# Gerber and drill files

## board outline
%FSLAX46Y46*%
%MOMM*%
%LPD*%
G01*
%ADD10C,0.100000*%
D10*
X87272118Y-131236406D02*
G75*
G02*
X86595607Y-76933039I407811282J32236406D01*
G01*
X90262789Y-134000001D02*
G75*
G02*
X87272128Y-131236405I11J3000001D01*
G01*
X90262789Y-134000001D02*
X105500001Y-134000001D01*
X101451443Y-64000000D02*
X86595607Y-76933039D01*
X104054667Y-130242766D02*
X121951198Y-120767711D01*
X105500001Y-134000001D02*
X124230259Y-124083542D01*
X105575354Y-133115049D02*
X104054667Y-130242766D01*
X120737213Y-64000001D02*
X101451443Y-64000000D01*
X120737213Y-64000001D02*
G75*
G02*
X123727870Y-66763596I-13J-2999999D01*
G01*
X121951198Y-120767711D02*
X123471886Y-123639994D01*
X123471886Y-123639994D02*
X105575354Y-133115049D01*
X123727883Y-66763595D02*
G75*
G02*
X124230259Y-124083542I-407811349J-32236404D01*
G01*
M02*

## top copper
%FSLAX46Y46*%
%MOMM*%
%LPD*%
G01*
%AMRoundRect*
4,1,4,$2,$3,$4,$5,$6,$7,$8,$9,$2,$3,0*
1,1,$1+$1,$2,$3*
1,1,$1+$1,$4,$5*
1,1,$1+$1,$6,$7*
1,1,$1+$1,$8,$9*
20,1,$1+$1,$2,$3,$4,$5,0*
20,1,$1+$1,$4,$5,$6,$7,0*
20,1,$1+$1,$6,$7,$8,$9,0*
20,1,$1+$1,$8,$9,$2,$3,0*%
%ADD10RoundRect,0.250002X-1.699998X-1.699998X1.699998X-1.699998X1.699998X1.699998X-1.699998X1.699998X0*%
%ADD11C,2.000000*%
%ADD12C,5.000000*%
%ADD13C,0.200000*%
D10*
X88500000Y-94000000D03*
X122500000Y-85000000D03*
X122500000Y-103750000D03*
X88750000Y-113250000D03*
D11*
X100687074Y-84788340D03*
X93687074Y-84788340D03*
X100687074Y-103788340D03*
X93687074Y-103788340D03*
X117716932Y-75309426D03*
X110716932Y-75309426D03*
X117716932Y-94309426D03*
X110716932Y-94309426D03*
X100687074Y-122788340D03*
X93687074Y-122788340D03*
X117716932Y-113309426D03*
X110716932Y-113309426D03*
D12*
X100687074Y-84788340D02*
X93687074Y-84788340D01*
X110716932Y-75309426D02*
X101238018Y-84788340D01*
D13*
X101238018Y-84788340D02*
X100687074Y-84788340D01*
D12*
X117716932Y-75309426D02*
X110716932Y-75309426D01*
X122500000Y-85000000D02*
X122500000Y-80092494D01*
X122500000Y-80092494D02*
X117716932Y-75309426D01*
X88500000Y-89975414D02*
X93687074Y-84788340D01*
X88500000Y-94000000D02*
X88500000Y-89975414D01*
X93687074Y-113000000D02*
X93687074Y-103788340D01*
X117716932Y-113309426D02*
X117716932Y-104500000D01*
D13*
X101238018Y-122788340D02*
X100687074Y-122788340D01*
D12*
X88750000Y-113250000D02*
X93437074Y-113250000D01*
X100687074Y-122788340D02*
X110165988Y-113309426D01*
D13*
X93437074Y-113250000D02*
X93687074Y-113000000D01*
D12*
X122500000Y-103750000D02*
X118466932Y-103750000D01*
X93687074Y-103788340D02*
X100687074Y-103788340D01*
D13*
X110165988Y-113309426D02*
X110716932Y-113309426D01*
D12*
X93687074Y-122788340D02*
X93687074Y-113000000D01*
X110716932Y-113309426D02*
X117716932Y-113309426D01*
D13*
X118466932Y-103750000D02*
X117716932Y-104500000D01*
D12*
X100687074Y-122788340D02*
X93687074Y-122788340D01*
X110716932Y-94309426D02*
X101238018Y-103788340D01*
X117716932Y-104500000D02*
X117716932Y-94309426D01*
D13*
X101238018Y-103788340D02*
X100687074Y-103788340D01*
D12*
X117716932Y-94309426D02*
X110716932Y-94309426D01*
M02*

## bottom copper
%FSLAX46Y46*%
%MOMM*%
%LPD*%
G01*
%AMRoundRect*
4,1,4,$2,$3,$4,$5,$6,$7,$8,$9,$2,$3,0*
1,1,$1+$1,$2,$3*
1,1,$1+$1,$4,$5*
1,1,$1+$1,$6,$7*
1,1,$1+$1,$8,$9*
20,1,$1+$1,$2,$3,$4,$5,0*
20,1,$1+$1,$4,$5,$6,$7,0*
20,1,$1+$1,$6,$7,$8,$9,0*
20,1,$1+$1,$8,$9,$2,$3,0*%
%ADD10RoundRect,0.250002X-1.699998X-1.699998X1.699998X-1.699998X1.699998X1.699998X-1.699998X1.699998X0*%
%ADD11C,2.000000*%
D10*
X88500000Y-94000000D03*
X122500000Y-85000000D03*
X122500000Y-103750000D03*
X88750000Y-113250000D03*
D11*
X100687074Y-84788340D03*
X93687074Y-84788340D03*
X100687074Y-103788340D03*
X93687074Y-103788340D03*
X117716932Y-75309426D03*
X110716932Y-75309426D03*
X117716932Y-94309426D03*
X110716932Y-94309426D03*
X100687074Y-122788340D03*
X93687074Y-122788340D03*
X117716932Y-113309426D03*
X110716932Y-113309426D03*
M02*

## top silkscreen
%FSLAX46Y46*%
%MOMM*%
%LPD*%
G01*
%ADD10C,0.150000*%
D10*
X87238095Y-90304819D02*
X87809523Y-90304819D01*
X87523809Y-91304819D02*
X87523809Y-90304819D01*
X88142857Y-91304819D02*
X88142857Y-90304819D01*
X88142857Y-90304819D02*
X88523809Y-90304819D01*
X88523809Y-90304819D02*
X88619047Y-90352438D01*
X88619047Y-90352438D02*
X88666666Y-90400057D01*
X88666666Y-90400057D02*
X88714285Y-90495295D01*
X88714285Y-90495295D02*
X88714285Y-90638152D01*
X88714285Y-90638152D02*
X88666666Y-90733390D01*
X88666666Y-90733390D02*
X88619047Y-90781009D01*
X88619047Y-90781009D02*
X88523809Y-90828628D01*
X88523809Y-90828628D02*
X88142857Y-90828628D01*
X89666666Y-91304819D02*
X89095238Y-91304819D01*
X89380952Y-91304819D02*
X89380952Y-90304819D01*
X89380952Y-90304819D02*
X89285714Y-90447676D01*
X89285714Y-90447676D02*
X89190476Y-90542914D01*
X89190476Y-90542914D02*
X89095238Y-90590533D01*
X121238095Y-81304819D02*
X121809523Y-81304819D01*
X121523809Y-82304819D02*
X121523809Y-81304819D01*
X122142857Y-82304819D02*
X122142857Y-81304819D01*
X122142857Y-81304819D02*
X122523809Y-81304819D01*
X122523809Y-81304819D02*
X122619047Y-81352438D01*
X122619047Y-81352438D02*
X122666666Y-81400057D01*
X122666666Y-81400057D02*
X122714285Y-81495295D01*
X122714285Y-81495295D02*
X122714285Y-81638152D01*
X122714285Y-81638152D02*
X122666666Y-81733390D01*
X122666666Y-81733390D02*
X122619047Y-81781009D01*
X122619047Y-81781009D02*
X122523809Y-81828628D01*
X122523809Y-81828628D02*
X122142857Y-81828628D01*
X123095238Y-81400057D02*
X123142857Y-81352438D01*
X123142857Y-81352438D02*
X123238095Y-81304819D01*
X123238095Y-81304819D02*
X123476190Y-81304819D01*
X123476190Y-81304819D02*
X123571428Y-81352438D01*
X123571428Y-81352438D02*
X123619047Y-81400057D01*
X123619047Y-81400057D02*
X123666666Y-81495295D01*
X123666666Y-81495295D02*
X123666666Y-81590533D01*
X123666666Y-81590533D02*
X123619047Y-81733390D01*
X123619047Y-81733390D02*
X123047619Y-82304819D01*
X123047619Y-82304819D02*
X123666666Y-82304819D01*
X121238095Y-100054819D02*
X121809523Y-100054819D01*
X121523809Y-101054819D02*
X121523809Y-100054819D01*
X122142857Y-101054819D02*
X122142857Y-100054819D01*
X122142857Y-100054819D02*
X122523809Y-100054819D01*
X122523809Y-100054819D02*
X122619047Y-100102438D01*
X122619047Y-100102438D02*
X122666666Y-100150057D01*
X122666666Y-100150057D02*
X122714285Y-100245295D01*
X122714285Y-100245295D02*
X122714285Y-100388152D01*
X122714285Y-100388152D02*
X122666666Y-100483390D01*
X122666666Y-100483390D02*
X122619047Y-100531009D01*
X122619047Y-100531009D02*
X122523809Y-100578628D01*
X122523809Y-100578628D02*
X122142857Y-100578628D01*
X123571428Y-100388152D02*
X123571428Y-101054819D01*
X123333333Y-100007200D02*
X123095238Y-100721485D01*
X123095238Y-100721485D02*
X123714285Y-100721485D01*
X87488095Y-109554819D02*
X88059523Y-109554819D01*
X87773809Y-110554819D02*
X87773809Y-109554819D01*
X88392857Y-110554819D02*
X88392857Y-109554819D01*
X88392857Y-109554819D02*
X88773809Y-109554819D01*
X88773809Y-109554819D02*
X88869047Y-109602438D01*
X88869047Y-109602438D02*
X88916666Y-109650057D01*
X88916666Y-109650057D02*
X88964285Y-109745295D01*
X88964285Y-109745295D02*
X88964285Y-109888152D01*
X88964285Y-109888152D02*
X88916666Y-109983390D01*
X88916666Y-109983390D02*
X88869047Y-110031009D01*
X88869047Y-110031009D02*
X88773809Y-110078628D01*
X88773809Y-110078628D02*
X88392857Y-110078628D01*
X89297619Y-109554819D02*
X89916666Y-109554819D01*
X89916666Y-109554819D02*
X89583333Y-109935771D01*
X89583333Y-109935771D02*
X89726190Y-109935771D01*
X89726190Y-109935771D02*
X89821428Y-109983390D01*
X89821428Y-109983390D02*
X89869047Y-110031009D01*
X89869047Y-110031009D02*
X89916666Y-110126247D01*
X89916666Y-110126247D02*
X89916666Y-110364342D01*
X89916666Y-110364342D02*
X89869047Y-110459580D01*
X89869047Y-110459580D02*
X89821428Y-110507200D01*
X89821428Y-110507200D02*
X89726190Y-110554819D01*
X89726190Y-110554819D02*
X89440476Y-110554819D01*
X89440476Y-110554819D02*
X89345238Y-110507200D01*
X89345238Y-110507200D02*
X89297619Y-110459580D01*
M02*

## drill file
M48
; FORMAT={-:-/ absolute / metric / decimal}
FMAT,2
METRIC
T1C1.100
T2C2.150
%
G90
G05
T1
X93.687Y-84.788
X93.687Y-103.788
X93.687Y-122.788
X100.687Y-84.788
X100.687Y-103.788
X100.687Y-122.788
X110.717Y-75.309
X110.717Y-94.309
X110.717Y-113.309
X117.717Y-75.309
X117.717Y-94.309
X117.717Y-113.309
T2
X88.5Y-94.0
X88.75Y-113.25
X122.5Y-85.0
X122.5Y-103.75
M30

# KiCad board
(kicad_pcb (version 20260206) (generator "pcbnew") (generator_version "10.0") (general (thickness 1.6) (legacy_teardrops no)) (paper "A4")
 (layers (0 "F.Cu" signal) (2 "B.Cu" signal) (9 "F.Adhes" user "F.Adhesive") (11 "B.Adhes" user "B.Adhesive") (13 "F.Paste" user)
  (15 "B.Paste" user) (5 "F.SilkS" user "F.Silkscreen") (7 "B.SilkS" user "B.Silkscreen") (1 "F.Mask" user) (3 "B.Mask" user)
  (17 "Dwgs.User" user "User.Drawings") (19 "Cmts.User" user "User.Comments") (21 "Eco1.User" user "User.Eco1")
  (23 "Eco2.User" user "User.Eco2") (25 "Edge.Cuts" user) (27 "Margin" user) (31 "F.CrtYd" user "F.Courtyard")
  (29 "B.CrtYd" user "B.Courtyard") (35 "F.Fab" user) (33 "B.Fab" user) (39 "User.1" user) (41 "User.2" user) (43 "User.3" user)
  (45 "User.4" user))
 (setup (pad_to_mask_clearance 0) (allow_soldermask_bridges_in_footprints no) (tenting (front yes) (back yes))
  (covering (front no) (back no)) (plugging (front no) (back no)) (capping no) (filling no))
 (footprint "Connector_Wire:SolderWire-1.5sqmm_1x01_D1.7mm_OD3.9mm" (layer "F.Cu") (at 88.5 94)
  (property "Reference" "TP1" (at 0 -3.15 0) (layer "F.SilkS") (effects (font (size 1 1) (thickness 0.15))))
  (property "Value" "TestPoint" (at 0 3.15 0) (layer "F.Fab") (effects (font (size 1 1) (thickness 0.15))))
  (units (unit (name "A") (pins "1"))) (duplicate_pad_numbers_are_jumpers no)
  (pad "1" thru_hole roundrect (at 0 0) (size 3.9 3.9) (drill 2.15) (layers "*.Cu" "*.Mask") (remove_unused_layers no)
   (roundrect_rratio 0.064103) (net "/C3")))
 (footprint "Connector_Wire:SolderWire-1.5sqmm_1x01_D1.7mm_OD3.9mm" (layer "F.Cu") (at 122.5 85)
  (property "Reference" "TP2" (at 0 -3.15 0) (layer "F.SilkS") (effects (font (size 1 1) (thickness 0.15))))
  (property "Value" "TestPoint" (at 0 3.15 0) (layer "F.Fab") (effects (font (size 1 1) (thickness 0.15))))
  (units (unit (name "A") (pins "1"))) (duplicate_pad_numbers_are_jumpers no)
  (pad "1" thru_hole roundrect (at 0 0) (size 3.9 3.9) (drill 2.15) (layers "*.Cu" "*.Mask") (remove_unused_layers no)
   (roundrect_rratio 0.064103) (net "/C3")))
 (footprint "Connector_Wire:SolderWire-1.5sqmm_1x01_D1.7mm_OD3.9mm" (layer "F.Cu") (at 122.5 103.75)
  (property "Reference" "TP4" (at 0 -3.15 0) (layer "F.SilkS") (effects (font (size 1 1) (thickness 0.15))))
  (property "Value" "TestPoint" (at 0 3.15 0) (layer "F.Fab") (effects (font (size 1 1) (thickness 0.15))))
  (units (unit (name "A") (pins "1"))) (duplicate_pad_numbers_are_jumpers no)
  (pad "1" thru_hole roundrect (at 0 0) (size 3.9 3.9) (drill 2.15) (layers "*.Cu" "*.Mask") (remove_unused_layers no)
   (roundrect_rratio 0.064103) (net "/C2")))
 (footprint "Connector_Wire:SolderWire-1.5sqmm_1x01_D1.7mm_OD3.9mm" (layer "F.Cu") (at 88.75 113.25)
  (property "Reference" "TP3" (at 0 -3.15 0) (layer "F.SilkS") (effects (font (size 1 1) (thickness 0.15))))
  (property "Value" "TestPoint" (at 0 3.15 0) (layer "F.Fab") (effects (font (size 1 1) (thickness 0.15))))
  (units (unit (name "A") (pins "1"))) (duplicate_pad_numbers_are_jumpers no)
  (pad "1" thru_hole roundrect (at 0 0) (size 3.9 3.9) (drill 2.15) (layers "*.Cu" "*.Mask") (remove_unused_layers no)
   (roundrect_rratio 0.064103) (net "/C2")))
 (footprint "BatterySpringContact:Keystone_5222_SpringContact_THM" (layer "B.Cu") (at 97.187074 84.78834 180)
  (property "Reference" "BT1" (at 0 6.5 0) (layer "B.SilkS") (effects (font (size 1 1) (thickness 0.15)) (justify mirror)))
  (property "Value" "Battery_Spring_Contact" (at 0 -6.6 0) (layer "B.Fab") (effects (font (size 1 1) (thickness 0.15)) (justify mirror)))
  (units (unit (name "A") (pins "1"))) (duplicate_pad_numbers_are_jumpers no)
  (pad "1" thru_hole circle (at -3.5 0 180) (size 2 2) (drill 1.1) (layers "*.Cu" "*.Mask") (remove_unused_layers no) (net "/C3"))
  (pad "1" thru_hole circle (at 3.5 0 180) (size 2 2) (drill 1.1) (layers "*.Cu" "*.Mask") (remove_unused_layers no) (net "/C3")))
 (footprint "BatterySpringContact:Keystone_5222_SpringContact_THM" (layer "B.Cu") (at 97.187074 103.78834 180)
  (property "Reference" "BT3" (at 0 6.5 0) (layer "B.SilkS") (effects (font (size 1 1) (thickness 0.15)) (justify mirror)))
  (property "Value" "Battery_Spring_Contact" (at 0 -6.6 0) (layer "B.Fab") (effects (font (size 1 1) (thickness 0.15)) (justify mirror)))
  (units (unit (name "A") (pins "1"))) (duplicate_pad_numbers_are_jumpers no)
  (pad "1" thru_hole circle (at -3.5 0 180) (size 2 2) (drill 1.1) (layers "*.Cu" "*.Mask") (remove_unused_layers no) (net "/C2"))
  (pad "1" thru_hole circle (at 3.5 0 180) (size 2 2) (drill 1.1) (layers "*.Cu" "*.Mask") (remove_unused_layers no) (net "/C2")))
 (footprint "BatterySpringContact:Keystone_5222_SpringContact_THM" (layer "B.Cu") (at 114.216932 75.309426 180)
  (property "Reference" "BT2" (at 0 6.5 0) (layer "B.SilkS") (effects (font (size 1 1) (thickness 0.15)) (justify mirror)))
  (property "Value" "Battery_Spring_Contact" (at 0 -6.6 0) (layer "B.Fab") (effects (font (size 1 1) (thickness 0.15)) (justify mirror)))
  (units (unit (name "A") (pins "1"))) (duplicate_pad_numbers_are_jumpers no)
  (pad "1" thru_hole circle (at -3.5 0 180) (size 2 2) (drill 1.1) (layers "*.Cu" "*.Mask") (remove_unused_layers no) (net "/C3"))
  (pad "1" thru_hole circle (at 3.5 0 180) (size 2 2) (drill 1.1) (layers "*.Cu" "*.Mask") (remove_unused_layers no) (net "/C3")))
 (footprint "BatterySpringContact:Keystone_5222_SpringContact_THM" (layer "B.Cu") (at 114.216932 94.309426 180)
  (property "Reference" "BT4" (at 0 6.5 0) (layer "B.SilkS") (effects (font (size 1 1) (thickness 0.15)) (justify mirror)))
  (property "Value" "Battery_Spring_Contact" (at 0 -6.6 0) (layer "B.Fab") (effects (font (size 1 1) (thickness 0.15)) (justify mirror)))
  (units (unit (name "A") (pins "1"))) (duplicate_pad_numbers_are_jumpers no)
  (pad "1" thru_hole circle (at -3.5 0 180) (size 2 2) (drill 1.1) (layers "*.Cu" "*.Mask") (remove_unused_layers no) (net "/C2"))
  (pad "1" thru_hole circle (at 3.5 0 180) (size 2 2) (drill 1.1) (layers "*.Cu" "*.Mask") (remove_unused_layers no) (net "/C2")))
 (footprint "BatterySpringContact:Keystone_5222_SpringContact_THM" (layer "B.Cu") (at 97.187074 122.78834 180)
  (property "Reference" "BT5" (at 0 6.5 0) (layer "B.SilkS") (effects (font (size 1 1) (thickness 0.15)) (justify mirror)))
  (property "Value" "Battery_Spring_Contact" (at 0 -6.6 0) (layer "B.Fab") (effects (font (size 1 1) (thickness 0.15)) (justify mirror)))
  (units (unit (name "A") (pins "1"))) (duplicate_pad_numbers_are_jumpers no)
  (pad "1" thru_hole circle (at -3.5 0 180) (size 2 2) (drill 1.1) (layers "*.Cu" "*.Mask") (remove_unused_layers no) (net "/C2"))
  (pad "1" thru_hole circle (at 3.5 0 180) (size 2 2) (drill 1.1) (layers "*.Cu" "*.Mask") (remove_unused_layers no) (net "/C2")))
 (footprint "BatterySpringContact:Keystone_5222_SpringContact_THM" (layer "B.Cu") (at 114.216932 113.309426 180)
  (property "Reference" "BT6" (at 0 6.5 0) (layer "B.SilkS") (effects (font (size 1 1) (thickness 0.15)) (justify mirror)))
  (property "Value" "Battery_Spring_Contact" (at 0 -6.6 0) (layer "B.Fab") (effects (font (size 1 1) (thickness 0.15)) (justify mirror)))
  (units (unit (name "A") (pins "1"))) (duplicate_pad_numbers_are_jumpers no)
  (pad "1" thru_hole circle (at -3.5 0 180) (size 2 2) (drill 1.1) (layers "*.Cu" "*.Mask") (remove_unused_layers no) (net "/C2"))
  (pad "1" thru_hole circle (at 3.5 0 180) (size 2 2) (drill 1.1) (layers "*.Cu" "*.Mask") (remove_unused_layers no) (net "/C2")))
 (gr_arc (start 87.272118 131.236406) (mid 86.031742 104.095961) (end 86.595607 76.933039) (stroke (width 0.1) (type default))
  (layer "Edge.Cuts"))
 (gr_arc (start 90.262789 134.000001) (mid 88.226767 133.203318) (end 87.272118 131.236406) (stroke (width 0.1) (type default))
  (layer "Edge.Cuts"))
 (gr_line (start 90.262789 134.000001) (end 105.500001 134.000001) (stroke (width 0.1) (type default)) (layer "Edge.Cuts"))
 (gr_line (start 101.451443 64) (end 86.595607 76.933039) (stroke (width 0.1) (type default)) (layer "Edge.Cuts"))
 (gr_line (start 104.054667 130.242766) (end 121.951198 120.767711) (stroke (width 0.1) (type default)) (layer "Edge.Cuts"))
 (gr_line (start 105.500001 134.000001) (end 124.230259 124.083542) (stroke (width 0.1) (type default)) (layer "Edge.Cuts"))
 (gr_line (start 105.575354 133.115049) (end 104.054667 130.242766) (stroke (width 0.1) (type default)) (layer "Edge.Cuts"))
 (gr_line (start 120.737213 64.000001) (end 101.451443 64) (stroke (width 0.1) (type default)) (layer "Edge.Cuts"))
 (gr_arc (start 120.737213 64.000001) (mid 122.773235 64.796684) (end 123.727883 66.763595) (stroke (width 0.1) (type default))
  (layer "Edge.Cuts"))
 (gr_line (start 121.951198 120.767711) (end 123.471886 123.639994) (stroke (width 0.1) (type default)) (layer "Edge.Cuts"))
 (gr_line (start 123.471886 123.639994) (end 105.575354 133.115049) (stroke (width 0.1) (type default)) (layer "Edge.Cuts"))
 (gr_arc (start 123.727883 66.763595) (mid 124.984289 95.414758) (end 124.230259 124.083542) (stroke (width 0.1) (type default))
  (layer "Edge.Cuts"))
 (segment (start 100.687074 84.78834) (end 93.687074 84.78834) (width 5) (layer "F.Cu") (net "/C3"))
 (segment (start 110.716932 75.309426) (end 101.238018 84.78834) (width 5) (layer "F.Cu") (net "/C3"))
 (segment (start 101.238018 84.78834) (end 100.687074 84.78834) (width 0.2) (layer "F.Cu") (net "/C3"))
 (segment (start 117.716932 75.309426) (end 110.716932 75.309426) (width 5) (layer "F.Cu") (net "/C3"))
 (segment (start 122.5 85) (end 122.5 80.092494) (width 5) (layer "F.Cu") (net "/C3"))
 (segment (start 122.5 80.092494) (end 117.716932 75.309426) (width 5) (layer "F.Cu") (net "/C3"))
 (segment (start 88.5 89.975414) (end 93.687074 84.78834) (width 5) (layer "F.Cu") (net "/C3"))
 (segment (start 88.5 94) (end 88.5 89.975414) (width 5) (layer "F.Cu") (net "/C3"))
 (segment (start 93.687074 113) (end 93.687074 103.78834) (width 5) (layer "F.Cu") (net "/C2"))
 (segment (start 117.716932 113.309426) (end 117.716932 104.5) (width 5) (layer "F.Cu") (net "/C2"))
 (segment (start 101.238018 122.78834) (end 100.687074 122.78834) (width 0.2) (layer "F.Cu") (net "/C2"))
 (segment (start 88.75 113.25) (end 93.437074 113.25) (width 5) (layer "F.Cu") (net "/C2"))
 (segment (start 100.687074 122.78834) (end 110.165988 113.309426) (width 5) (layer "F.Cu") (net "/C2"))
 (segment (start 93.437074 113.25) (end 93.687074 113) (width 0.2) (layer "F.Cu") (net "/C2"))
 (segment (start 122.5 103.75) (end 118.466932 103.75) (width 5) (layer "F.Cu") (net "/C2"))
 (segment (start 93.687074 103.78834) (end 100.687074 103.78834) (width 5) (layer "F.Cu") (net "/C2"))
 (segment (start 110.165988 113.309426) (end 110.716932 113.309426) (width 0.2) (layer "F.Cu") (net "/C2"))
 (segment (start 93.687074 122.78834) (end 93.687074 113) (width 5) (layer "F.Cu") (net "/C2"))
 (segment (start 110.716932 113.309426) (end 117.716932 113.309426) (width 5) (layer "F.Cu") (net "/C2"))
 (segment (start 118.466932 103.75) (end 117.716932 104.5) (width 0.2) (layer "F.Cu") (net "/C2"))
 (segment (start 100.687074 122.78834) (end 93.687074 122.78834) (width 5) (layer "F.Cu") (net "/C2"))
 (segment (start 110.716932 94.309426) (end 101.238018 103.78834) (width 5) (layer "F.Cu") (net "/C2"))
 (segment (start 117.716932 104.5) (end 117.716932 94.309426) (width 5) (layer "F.Cu") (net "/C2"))
 (segment (start 101.238018 103.78834) (end 100.687074 103.78834) (width 0.2) (layer "F.Cu") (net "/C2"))
 (segment (start 117.716932 94.309426) (end 110.716932 94.309426) (width 5) (layer "F.Cu") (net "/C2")))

